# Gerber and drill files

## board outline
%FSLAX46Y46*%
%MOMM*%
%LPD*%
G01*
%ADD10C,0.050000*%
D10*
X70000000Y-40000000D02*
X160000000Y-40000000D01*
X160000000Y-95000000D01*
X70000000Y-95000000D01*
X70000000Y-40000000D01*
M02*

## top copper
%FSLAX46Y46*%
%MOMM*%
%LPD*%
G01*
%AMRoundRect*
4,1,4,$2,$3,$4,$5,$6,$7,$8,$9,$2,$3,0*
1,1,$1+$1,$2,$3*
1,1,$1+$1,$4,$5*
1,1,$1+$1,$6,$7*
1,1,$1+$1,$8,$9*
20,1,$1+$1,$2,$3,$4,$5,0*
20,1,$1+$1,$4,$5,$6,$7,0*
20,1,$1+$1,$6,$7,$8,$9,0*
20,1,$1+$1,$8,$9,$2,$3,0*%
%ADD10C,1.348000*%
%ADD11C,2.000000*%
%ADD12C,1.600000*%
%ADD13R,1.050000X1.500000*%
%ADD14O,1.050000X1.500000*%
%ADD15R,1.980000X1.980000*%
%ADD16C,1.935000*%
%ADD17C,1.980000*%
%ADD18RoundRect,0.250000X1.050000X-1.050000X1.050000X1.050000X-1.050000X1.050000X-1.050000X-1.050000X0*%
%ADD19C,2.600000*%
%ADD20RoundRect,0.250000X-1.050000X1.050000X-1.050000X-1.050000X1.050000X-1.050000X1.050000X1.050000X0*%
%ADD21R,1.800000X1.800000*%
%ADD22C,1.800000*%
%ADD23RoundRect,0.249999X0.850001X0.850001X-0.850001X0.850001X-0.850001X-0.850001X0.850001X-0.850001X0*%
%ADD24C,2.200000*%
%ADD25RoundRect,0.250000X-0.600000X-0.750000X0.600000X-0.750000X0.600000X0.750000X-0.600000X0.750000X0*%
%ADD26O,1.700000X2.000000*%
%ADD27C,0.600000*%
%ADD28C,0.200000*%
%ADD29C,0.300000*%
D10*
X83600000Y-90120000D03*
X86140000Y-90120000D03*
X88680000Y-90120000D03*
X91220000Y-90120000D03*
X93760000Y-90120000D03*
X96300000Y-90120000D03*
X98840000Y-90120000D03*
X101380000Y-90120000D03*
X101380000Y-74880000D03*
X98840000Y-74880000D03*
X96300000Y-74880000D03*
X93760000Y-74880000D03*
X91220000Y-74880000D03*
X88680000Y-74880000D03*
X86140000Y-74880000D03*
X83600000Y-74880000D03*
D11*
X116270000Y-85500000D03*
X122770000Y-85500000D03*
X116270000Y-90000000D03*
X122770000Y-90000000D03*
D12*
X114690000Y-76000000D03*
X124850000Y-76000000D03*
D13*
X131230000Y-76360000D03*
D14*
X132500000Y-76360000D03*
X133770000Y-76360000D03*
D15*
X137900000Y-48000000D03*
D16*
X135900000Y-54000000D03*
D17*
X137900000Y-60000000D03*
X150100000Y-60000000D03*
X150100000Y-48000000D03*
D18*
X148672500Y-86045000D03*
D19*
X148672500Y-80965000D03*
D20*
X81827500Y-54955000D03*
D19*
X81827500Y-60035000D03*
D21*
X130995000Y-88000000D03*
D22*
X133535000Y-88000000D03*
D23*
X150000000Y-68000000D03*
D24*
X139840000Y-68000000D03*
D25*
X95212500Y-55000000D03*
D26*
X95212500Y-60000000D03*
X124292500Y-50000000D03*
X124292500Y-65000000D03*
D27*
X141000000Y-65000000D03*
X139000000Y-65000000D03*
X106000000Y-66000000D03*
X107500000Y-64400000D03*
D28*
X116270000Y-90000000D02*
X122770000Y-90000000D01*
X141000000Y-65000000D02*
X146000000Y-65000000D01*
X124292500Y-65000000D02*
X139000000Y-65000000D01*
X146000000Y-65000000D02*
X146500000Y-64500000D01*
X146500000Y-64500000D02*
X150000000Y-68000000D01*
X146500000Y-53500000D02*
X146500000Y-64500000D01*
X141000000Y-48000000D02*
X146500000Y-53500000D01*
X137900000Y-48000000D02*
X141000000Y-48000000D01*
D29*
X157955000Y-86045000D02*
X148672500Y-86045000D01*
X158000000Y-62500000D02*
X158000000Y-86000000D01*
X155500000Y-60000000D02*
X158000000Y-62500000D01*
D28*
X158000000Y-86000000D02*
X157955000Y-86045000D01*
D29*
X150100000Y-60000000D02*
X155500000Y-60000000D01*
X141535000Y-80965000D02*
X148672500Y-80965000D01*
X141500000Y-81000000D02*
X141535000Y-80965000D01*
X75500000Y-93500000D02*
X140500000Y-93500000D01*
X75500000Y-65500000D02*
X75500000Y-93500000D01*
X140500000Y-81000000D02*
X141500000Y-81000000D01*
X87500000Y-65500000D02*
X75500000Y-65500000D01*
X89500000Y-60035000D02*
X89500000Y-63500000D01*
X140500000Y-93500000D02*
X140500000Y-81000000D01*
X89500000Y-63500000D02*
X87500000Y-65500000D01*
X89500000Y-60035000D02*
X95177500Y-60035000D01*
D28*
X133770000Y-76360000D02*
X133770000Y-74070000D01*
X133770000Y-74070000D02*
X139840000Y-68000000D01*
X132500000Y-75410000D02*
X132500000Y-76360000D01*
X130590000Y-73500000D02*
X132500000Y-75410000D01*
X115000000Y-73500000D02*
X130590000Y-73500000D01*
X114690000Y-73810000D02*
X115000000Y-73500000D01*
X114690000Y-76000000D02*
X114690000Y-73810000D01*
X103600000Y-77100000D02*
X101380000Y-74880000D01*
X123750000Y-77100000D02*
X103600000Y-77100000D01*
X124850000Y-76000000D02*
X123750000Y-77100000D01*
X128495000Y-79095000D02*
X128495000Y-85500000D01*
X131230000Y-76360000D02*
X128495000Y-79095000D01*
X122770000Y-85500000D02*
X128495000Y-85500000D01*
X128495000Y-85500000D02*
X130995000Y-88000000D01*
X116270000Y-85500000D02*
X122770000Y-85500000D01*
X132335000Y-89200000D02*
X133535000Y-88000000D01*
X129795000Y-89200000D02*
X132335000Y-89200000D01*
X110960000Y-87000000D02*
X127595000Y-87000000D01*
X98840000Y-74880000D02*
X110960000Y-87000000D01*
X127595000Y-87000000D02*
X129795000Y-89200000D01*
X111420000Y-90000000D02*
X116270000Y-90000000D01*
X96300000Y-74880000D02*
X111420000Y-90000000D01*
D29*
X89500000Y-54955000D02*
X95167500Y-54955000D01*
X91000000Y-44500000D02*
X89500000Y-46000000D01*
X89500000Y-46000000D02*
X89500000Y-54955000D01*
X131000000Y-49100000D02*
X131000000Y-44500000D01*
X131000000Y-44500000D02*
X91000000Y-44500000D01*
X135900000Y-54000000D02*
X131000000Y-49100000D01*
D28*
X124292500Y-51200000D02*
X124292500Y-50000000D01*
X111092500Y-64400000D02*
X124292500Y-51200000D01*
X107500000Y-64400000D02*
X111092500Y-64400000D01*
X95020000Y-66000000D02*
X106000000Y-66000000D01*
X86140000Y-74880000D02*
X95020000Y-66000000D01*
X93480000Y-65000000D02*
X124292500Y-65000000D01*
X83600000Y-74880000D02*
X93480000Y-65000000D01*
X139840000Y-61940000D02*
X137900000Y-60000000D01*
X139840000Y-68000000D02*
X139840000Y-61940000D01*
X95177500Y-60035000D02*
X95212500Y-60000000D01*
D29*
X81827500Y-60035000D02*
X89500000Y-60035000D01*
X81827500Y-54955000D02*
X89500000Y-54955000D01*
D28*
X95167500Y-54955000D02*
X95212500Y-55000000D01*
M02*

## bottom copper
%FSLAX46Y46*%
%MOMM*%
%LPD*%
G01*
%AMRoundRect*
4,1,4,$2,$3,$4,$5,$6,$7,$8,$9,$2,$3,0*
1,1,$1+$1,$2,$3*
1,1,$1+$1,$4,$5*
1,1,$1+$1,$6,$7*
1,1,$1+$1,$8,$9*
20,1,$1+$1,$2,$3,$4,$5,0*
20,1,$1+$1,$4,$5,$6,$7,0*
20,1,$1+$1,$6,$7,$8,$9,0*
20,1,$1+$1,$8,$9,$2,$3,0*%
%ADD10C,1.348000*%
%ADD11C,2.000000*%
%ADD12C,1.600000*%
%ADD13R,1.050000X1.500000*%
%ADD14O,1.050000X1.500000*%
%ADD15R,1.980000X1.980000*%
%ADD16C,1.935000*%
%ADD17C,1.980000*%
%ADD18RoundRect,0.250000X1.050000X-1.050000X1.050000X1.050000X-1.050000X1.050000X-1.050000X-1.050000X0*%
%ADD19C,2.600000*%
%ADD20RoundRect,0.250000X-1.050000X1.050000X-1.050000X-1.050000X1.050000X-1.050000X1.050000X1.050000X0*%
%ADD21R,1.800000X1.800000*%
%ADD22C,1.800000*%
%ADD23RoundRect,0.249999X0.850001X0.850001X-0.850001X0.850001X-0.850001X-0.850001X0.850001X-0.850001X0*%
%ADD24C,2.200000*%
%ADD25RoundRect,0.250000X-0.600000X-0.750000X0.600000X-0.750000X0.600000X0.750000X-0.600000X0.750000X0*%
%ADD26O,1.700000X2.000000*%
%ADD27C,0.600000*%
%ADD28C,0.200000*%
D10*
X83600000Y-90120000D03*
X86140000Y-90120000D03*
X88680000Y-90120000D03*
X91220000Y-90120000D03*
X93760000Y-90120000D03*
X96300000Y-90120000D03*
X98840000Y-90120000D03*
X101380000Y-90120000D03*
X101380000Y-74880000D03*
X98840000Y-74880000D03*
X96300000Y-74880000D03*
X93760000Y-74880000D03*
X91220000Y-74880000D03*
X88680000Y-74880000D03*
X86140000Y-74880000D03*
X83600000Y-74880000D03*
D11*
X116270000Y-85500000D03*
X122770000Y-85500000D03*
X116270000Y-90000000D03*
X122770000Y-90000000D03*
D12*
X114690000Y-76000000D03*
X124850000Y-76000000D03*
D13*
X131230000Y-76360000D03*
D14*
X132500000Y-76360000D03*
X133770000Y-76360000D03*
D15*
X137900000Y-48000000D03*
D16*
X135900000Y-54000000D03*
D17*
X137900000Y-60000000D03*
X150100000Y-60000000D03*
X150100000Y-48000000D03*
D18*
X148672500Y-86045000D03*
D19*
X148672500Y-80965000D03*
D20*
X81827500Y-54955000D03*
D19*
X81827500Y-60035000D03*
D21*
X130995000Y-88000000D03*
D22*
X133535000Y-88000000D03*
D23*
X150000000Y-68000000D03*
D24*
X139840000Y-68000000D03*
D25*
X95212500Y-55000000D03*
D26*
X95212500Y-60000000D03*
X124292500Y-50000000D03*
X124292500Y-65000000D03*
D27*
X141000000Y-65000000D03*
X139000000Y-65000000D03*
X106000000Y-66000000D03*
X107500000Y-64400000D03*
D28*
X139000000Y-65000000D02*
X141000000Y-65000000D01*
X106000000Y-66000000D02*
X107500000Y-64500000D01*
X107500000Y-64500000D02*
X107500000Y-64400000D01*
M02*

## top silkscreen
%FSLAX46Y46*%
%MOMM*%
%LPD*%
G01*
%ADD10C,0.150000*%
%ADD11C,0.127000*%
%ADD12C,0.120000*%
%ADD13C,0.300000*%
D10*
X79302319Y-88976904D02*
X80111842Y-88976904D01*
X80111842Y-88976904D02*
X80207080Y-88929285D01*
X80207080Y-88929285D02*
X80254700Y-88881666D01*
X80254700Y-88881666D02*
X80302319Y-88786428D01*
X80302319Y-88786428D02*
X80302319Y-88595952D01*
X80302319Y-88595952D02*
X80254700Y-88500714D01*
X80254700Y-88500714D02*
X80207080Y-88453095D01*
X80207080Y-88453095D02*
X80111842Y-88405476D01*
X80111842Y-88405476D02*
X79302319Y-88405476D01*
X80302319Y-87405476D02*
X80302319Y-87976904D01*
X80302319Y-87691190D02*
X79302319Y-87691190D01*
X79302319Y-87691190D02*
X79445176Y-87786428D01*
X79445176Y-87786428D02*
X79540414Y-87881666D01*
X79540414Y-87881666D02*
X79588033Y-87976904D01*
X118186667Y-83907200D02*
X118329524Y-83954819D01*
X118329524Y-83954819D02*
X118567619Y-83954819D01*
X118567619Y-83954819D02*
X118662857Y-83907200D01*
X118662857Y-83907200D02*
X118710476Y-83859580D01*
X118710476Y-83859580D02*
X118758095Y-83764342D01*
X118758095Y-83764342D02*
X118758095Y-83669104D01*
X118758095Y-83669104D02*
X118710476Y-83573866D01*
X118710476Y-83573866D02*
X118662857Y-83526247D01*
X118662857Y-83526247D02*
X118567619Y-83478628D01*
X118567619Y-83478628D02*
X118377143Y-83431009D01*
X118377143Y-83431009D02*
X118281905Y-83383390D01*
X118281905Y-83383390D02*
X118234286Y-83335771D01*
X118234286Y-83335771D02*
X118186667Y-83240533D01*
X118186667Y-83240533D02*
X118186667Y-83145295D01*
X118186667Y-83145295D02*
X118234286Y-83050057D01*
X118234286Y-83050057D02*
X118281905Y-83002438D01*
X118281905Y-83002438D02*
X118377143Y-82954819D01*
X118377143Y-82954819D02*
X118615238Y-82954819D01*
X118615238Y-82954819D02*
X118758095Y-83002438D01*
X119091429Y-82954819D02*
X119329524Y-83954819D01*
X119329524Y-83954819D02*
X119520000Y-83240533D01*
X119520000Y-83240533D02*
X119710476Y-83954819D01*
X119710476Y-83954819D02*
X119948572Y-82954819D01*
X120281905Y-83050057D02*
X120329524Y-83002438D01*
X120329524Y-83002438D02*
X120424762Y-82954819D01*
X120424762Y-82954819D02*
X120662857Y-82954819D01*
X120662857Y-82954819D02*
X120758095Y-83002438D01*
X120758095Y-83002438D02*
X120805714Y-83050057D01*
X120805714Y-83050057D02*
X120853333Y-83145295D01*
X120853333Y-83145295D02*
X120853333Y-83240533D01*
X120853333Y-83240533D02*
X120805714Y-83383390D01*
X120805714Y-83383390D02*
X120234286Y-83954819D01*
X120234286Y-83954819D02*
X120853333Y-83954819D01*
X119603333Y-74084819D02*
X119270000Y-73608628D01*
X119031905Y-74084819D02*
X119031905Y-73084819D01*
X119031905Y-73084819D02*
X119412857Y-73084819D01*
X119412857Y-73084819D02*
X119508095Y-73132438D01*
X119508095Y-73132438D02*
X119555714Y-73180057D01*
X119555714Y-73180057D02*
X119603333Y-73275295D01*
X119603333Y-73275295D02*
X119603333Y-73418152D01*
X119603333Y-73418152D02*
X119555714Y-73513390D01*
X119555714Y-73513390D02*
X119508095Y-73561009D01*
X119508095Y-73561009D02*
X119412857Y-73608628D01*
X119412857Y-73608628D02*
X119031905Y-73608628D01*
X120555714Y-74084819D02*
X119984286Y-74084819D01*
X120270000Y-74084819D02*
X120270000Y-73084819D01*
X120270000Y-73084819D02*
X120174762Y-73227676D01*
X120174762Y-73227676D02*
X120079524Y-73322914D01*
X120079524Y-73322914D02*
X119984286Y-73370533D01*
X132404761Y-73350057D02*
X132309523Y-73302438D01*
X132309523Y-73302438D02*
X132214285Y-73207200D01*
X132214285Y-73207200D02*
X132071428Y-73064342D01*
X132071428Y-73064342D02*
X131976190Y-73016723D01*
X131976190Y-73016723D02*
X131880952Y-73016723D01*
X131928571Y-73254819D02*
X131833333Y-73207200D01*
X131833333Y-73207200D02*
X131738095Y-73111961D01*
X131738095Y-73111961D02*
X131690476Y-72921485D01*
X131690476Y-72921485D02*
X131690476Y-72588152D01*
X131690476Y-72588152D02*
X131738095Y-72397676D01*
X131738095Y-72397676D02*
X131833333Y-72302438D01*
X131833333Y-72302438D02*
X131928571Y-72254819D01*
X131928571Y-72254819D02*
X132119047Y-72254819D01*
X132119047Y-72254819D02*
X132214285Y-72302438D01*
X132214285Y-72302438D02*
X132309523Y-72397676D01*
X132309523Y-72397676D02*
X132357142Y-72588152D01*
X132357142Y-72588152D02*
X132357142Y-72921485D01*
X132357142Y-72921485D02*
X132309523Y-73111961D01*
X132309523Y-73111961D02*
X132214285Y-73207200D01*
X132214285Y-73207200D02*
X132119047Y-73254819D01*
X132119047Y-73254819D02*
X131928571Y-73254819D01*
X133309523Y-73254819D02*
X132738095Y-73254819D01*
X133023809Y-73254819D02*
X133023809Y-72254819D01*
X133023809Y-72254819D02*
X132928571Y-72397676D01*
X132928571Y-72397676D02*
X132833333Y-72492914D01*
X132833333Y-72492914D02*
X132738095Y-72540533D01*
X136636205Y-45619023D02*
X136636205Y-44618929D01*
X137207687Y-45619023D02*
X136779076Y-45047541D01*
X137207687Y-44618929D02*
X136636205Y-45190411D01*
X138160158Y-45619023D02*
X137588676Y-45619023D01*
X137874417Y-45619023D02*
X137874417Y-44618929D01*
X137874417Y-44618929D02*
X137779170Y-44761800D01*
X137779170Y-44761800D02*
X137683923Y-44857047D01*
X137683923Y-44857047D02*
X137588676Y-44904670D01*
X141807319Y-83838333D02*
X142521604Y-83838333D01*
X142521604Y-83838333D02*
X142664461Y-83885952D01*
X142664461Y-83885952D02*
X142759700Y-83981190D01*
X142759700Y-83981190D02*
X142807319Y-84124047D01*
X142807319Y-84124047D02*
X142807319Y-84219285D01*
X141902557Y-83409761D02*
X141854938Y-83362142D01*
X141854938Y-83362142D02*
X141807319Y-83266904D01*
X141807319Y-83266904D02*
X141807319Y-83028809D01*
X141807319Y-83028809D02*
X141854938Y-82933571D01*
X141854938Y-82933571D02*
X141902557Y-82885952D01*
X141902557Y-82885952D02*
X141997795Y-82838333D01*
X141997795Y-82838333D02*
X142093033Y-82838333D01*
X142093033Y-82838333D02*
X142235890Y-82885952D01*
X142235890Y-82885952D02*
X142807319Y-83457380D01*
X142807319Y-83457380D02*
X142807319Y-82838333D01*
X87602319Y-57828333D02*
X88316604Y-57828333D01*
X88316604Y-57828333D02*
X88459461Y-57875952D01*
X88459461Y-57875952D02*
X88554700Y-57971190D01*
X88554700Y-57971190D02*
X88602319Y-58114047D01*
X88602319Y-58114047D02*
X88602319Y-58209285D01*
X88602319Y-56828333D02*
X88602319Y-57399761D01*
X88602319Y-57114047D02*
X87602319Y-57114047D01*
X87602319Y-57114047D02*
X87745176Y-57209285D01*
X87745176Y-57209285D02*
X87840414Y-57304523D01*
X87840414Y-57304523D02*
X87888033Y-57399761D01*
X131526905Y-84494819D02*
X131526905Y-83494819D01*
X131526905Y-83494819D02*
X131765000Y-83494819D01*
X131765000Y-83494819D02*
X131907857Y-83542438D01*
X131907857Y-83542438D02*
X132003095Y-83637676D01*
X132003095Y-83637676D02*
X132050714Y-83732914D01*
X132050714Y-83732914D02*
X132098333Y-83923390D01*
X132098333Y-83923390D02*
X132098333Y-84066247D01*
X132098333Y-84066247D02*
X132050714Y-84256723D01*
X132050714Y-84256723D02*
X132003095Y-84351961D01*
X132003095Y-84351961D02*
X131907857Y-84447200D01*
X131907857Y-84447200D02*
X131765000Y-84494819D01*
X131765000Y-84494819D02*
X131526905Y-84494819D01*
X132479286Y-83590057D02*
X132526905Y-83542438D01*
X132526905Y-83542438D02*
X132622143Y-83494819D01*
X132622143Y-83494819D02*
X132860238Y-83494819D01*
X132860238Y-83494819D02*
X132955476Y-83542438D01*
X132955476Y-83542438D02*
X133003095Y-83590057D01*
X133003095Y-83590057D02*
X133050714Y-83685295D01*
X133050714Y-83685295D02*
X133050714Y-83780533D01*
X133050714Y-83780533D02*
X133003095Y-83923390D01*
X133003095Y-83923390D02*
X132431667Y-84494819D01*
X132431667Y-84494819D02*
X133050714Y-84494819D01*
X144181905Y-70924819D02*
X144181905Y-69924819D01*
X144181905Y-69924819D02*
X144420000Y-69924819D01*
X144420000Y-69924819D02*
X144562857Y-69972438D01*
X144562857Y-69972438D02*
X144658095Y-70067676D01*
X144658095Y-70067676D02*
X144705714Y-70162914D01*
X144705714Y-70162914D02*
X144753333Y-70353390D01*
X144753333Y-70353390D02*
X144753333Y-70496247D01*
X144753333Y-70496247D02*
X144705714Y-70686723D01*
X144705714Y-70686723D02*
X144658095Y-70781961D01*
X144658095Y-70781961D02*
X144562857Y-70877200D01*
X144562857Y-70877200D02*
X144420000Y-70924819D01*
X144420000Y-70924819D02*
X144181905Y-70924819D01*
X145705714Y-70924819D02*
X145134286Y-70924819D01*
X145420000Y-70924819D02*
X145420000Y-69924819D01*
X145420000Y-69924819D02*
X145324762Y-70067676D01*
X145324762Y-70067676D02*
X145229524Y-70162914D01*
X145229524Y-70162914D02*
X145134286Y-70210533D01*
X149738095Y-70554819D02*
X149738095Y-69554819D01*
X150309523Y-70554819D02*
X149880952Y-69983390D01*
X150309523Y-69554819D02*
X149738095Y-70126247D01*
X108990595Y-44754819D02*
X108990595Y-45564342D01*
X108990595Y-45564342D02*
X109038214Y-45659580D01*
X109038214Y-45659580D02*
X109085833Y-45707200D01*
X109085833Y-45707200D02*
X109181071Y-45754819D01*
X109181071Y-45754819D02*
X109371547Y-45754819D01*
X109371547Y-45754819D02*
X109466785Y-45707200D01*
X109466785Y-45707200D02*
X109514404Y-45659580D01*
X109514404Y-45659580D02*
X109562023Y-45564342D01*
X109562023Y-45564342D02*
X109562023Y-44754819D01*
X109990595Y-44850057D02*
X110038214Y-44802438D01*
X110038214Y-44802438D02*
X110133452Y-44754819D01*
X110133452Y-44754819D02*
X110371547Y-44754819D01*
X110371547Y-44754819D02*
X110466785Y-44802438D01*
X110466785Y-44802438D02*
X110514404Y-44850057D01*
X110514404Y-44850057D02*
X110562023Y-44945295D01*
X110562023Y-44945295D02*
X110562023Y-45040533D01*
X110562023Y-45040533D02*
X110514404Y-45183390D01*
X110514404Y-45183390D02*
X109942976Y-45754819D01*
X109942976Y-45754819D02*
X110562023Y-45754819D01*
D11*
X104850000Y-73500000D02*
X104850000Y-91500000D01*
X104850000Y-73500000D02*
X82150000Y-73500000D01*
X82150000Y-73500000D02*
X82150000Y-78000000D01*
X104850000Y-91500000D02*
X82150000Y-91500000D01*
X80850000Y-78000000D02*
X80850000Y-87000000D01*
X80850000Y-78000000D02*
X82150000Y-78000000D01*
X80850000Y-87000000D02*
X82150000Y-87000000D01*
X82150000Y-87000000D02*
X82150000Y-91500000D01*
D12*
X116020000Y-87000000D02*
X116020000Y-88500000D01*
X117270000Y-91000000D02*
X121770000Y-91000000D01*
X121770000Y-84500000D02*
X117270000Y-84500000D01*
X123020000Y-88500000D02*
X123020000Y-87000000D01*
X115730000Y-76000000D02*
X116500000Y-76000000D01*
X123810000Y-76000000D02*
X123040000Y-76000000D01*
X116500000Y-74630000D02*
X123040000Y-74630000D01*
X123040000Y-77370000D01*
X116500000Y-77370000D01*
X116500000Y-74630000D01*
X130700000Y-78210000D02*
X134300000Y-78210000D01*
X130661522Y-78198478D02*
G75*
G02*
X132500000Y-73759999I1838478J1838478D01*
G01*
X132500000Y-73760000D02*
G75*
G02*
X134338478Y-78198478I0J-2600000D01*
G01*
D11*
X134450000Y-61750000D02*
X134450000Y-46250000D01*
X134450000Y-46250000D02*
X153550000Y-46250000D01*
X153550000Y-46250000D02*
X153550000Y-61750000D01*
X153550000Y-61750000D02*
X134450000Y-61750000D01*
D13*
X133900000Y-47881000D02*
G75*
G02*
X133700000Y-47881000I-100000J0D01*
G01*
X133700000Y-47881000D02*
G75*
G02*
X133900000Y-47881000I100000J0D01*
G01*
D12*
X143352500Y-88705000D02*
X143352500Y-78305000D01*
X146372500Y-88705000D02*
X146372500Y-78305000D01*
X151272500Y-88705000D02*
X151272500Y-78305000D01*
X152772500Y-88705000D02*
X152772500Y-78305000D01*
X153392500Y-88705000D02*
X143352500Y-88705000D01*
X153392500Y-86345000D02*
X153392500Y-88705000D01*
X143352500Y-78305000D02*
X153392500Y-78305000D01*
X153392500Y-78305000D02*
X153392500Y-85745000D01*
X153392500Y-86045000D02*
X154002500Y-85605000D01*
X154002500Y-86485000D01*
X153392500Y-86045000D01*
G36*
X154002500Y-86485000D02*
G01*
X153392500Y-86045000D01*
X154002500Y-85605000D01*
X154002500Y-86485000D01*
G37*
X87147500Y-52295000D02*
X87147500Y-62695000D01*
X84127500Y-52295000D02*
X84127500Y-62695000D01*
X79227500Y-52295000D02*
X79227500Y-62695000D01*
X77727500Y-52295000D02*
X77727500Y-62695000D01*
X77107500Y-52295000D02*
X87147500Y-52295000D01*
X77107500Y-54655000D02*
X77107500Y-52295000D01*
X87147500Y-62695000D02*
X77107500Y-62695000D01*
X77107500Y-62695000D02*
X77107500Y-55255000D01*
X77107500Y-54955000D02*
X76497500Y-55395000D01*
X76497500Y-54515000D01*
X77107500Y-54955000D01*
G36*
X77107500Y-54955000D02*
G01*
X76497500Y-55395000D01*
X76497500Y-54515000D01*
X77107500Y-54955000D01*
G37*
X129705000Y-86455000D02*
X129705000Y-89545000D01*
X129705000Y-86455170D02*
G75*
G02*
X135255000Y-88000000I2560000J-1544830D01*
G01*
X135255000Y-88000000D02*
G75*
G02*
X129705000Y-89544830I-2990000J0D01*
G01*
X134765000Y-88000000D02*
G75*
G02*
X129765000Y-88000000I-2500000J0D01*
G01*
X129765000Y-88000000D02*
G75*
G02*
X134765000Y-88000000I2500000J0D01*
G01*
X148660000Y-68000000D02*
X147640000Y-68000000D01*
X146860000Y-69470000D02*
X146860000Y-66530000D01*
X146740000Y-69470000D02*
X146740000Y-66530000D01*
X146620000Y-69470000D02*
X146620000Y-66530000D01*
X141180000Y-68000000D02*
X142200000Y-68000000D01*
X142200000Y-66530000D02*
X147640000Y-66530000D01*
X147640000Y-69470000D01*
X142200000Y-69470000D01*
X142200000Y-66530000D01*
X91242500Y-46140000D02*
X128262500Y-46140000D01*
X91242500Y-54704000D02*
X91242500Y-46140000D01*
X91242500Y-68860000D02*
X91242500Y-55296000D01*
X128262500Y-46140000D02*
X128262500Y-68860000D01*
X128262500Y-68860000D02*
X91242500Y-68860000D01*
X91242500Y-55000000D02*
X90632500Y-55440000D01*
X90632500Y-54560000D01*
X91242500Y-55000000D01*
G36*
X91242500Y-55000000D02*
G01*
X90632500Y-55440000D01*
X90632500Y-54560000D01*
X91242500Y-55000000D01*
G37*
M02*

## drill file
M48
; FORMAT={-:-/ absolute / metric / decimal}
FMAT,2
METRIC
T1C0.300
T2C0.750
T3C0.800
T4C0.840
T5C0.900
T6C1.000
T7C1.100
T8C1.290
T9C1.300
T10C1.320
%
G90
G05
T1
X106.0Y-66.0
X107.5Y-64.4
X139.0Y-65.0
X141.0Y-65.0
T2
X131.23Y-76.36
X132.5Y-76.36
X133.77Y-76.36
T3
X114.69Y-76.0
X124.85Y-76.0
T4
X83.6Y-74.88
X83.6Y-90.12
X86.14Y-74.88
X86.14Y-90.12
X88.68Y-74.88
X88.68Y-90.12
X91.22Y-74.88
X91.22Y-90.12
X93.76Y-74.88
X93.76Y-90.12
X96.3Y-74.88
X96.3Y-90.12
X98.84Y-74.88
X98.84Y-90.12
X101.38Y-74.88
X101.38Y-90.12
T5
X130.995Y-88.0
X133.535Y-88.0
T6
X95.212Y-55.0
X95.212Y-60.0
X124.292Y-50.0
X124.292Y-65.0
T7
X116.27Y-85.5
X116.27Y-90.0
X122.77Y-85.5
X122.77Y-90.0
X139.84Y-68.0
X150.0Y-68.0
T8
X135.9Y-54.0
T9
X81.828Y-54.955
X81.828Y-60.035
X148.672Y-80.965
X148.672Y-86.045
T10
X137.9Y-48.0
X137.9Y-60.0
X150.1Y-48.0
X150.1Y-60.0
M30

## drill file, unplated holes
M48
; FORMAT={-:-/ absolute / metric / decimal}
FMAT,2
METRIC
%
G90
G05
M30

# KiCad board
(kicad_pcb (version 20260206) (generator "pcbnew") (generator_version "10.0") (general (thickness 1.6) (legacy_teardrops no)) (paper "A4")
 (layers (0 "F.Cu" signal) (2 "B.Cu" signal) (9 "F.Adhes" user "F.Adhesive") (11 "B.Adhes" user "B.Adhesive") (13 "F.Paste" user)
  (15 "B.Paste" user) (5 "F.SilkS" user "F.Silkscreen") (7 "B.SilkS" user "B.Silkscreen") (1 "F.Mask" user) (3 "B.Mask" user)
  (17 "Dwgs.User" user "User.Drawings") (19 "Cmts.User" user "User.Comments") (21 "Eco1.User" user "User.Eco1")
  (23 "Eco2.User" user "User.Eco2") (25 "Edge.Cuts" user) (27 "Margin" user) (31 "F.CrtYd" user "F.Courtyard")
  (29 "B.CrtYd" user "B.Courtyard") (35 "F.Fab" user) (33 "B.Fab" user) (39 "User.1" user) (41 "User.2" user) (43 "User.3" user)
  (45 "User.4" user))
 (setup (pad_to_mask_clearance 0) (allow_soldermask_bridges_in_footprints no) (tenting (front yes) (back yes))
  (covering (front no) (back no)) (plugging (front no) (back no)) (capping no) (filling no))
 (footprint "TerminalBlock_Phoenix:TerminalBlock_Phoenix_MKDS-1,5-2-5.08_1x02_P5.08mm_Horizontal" (layer "F.Cu") (at 148.6725 86.045 90)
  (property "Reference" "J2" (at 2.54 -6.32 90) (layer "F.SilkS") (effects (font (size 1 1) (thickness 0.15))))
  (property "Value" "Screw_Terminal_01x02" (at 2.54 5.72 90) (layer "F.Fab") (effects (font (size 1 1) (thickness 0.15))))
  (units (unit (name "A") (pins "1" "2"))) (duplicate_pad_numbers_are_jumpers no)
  (fp_line (start 7.74 -5.32) (end 7.74 4.72) (stroke (width 0.12) (type solid)) (layer "F.SilkS"))
  (fp_line (start -2.66 -5.32) (end 7.74 -5.32) (stroke (width 0.12) (type solid)) (layer "F.SilkS"))
  (fp_line (start -2.66 -2.3) (end 7.74 -2.3) (stroke (width 0.12) (type solid)) (layer "F.SilkS"))
  (fp_line (start -2.66 2.6) (end 7.74 2.6) (stroke (width 0.12) (type solid)) (layer "F.SilkS"))
  (fp_line (start -2.66 4.1) (end 7.74 4.1) (stroke (width 0.12) (type solid)) (layer "F.SilkS"))
  (fp_line (start 7.74 4.72) (end 0.3 4.72) (stroke (width 0.12) (type solid)) (layer "F.SilkS"))
  (fp_line (start -0.3 4.72) (end -2.66 4.72) (stroke (width 0.12) (type solid)) (layer "F.SilkS"))
  (fp_line (start -2.66 4.72) (end -2.66 -5.32) (stroke (width 0.12) (type solid)) (layer "F.SilkS"))
  (fp_poly (pts (xy 0 4.72) (xy 0.44 5.33) (xy -0.44 5.33)) (stroke (width 0.12) (type solid)) (fill yes) (layer "F.SilkS"))
  (pad "1" thru_hole roundrect (at 0 0 90) (size 2.6 2.6) (drill 1.3) (layers "*.Cu" "*.Mask") (remove_unused_layers no)
   (roundrect_rratio 0.096154) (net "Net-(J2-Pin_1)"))
  (pad "2" thru_hole circle (at 5.08 0 90) (size 2.6 2.6) (drill 1.3) (layers "*.Cu" "*.Mask") (remove_unused_layers no)
   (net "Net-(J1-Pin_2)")))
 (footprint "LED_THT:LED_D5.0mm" (layer "F.Cu") (at 130.995 88)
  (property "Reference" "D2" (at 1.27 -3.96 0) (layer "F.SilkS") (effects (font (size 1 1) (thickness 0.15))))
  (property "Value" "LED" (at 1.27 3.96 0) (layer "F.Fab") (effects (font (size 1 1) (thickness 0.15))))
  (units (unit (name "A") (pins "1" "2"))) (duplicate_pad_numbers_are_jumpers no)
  (fp_line (start -1.29 -1.545) (end -1.29 1.545) (stroke (width 0.12) (type solid)) (layer "F.SilkS"))
  (fp_arc (start -1.29 -1.54483) (mid 2.071779 -2.880495) (end 4.26 0) (stroke (width 0.12) (type solid)) (layer "F.SilkS"))
  (fp_arc (start 4.26 0) (mid 2.071779 2.880495) (end -1.29 1.54483) (stroke (width 0.12) (type solid)) (layer "F.SilkS"))
  (fp_circle (center 1.27 0) (end 3.77 0) (stroke (width 0.12) (type solid)) (fill no) (layer "F.SilkS"))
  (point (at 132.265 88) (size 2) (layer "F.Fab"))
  (pad "1" thru_hole rect (at 0 0) (size 1.8 1.8) (drill 0.9) (layers "*.Cu" "*.Mask") (remove_unused_layers no) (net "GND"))
  (pad "2" thru_hole circle (at 2.54 0) (size 1.8 1.8) (drill 0.9) (layers "*.Cu" "*.Mask") (remove_unused_layers no) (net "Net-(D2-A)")))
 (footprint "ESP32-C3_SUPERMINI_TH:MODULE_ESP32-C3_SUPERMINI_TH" (layer "F.Cu") (at 93.5 82.5 90)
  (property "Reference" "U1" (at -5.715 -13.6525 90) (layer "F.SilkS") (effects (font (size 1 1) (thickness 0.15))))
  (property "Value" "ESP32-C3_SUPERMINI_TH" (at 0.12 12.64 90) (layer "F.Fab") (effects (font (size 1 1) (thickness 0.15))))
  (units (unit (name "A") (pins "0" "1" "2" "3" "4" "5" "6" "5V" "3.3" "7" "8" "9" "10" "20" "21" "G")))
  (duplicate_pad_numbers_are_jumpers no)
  (fp_line (start 4.5 -12.65) (end -4.5 -12.65) (stroke (width 0.127) (type solid)) (layer "F.SilkS"))
  (fp_line (start 4.5 -12.65) (end 4.5 -11.35) (stroke (width 0.127) (type solid)) (layer "F.SilkS"))
  (fp_line (start -4.5 -12.65) (end -4.5 -11.35) (stroke (width 0.127) (type solid)) (layer "F.SilkS"))
  (fp_line (start 9 -11.35) (end 4.5 -11.35) (stroke (width 0.127) (type solid)) (layer "F.SilkS"))
  (fp_line (start -4.5 -11.35) (end -9 -11.35) (stroke (width 0.127) (type solid)) (layer "F.SilkS"))
  (fp_line (start 9 11.35) (end 9 -11.35) (stroke (width 0.127) (type solid)) (layer "F.SilkS"))
  (fp_line (start 9 11.35) (end -9 11.35) (stroke (width 0.127) (type solid)) (layer "F.SilkS"))
  (fp_line (start -9 11.35) (end -9 -11.35) (stroke (width 0.127) (type solid)) (layer "F.SilkS"))
  (pad "0" thru_hole circle (at 7.62 7.88 90) (size 1.348 1.348) (drill 0.84) (layers "*.Cu" "*.Mask") (remove_unused_layers no)
   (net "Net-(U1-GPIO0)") (solder_mask_margin 0.102))
  (pad "1" thru_hole circle (at 7.62 5.34 90) (size 1.348 1.348) (drill 0.84) (layers "*.Cu" "*.Mask") (remove_unused_layers no)
   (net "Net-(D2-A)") (solder_mask_margin 0.102))
  (pad "2" thru_hole circle (at 7.62 2.8 90) (size 1.348 1.348) (drill 0.84) (layers "*.Cu" "*.Mask") (remove_unused_layers no)
   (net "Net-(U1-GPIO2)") (solder_mask_margin 0.102))
  (pad "3" thru_hole circle (at 7.62 0.26 90) (size 1.348 1.348) (drill 0.84) (layers "*.Cu" "*.Mask") (remove_unused_layers no)
   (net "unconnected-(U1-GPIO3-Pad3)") (solder_mask_margin 0.102))
  (pad "3.3" thru_hole circle (at 7.62 -4.82 90) (size 1.348 1.348) (drill 0.84) (layers "*.Cu" "*.Mask") (remove_unused_layers no)
   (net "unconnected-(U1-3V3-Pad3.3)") (solder_mask_margin 0.102))
  (pad "4" thru_hole circle (at 7.62 -2.28 90) (size 1.348 1.348) (drill 0.84) (layers "*.Cu" "*.Mask") (remove_unused_layers no)
   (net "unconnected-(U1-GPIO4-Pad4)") (solder_mask_margin 0.102))
  (pad "5" thru_hole circle (at -7.62 -9.9 90) (size 1.348 1.348) (drill 0.84) (layers "*.Cu" "*.Mask") (remove_unused_layers no)
   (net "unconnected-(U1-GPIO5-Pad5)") (solder_mask_margin 0.102))
  (pad "5V" thru_hole circle (at 7.62 -9.9 90) (size 1.348 1.348) (drill 0.84) (layers "*.Cu" "*.Mask") (remove_unused_layers no)
   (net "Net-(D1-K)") (solder_mask_margin 0.102))
  (pad "6" thru_hole circle (at -7.62 -7.36 90) (size 1.348 1.348) (drill 0.84) (layers "*.Cu" "*.Mask") (remove_unused_layers no)
   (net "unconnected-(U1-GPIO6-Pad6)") (solder_mask_margin 0.102))
  (pad "7" thru_hole circle (at -7.62 -4.82 90) (size 1.348 1.348) (drill 0.84) (layers "*.Cu" "*.Mask") (remove_unused_layers no)
   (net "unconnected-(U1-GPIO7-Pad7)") (solder_mask_margin 0.102))
  (pad "8" thru_hole circle (at -7.62 -2.28 90) (size 1.348 1.348) (drill 0.84) (layers "*.Cu" "*.Mask") (remove_unused_layers no)
   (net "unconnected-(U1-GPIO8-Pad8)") (solder_mask_margin 0.102))
  (pad "9" thru_hole circle (at -7.62 0.26 90) (size 1.348 1.348) (drill 0.84) (layers "*.Cu" "*.Mask") (remove_unused_layers no)
   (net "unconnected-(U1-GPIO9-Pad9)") (solder_mask_margin 0.102))
  (pad "10" thru_hole circle (at -7.62 2.8 90) (size 1.348 1.348) (drill 0.84) (layers "*.Cu" "*.Mask") (remove_unused_layers no)
   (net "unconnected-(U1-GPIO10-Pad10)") (solder_mask_margin 0.102))
  (pad "20" thru_hole circle (at -7.62 5.34 90) (size 1.348 1.348) (drill 0.84) (layers "*.Cu" "*.Mask") (remove_unused_layers no)
   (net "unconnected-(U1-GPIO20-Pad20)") (solder_mask_margin 0.102))
  (pad "21" thru_hole circle (at -7.62 7.88 90) (size 1.348 1.348) (drill 0.84) (layers "*.Cu" "*.Mask") (remove_unused_layers no)
   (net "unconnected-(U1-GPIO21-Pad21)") (solder_mask_margin 0.102))
  (pad "G" thru_hole circle (at 7.62 -7.36 90) (size 1.348 1.348) (drill 0.84) (layers "*.Cu" "*.Mask") (remove_unused_layers no)
   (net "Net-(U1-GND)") (solder_mask_margin 0.102)))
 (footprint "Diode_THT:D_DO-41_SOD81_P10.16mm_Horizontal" (layer "F.Cu") (at 150 68 180)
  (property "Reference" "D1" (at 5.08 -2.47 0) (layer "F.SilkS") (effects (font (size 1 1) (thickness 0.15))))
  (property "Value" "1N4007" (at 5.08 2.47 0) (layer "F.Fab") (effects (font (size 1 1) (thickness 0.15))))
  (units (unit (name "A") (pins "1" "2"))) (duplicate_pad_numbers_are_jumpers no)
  (fp_line (start 8.82 0) (end 7.8 0) (stroke (width 0.12) (type solid)) (layer "F.SilkS"))
  (fp_line (start 3.38 -1.47) (end 3.38 1.47) (stroke (width 0.12) (type solid)) (layer "F.SilkS"))
  (fp_line (start 3.26 -1.47) (end 3.26 1.47) (stroke (width 0.12) (type solid)) (layer "F.SilkS"))
  (fp_line (start 3.14 -1.47) (end 3.14 1.47) (stroke (width 0.12) (type solid)) (layer "F.SilkS"))
  (fp_line (start 1.34 0) (end 2.36 0) (stroke (width 0.12) (type solid)) (layer "F.SilkS"))
  (fp_rect (start 2.36 -1.47) (end 7.8 1.47) (stroke (width 0.12) (type solid)) (fill no) (layer "F.SilkS"))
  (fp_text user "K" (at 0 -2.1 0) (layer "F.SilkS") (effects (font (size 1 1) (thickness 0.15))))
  (pad "1" thru_hole roundrect (at 0 0 180) (size 2.2 2.2) (drill 1.1) (layers "*.Cu" "*.Mask") (remove_unused_layers no)
   (roundrect_rratio 0.113636) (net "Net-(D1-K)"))
  (pad "2" thru_hole circle (at 10.16 0 180) (size 2.2 2.2) (drill 1.1) (layers "*.Cu" "*.Mask") (remove_unused_layers no)
   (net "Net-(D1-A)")))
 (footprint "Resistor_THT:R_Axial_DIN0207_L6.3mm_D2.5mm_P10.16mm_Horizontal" (layer "F.Cu") (at 114.69 76)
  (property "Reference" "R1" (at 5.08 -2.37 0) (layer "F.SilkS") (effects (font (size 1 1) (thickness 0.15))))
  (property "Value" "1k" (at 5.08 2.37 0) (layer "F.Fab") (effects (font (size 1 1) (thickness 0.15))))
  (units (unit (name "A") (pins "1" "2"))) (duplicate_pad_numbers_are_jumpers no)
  (fp_line (start 1.04 0) (end 1.81 0) (stroke (width 0.12) (type solid)) (layer "F.SilkS"))
  (fp_line (start 9.12 0) (end 8.35 0) (stroke (width 0.12) (type solid)) (layer "F.SilkS"))
  (fp_rect (start 1.81 -1.37) (end 8.35 1.37) (stroke (width 0.12) (type solid)) (fill no) (layer "F.SilkS"))
  (pad "1" thru_hole circle (at 0 0) (size 1.6 1.6) (drill 0.8) (layers "*.Cu" "*.Mask") (remove_unused_layers no) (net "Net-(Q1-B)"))
  (pad "2" thru_hole circle (at 10.16 0) (size 1.6 1.6) (drill 0.8) (layers "*.Cu" "*.Mask") (remove_unused_layers no)
   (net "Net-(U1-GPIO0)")))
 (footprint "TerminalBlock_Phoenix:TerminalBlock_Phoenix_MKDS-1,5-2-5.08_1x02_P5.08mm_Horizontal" (layer "F.Cu") (at 81.8275 54.955 -90)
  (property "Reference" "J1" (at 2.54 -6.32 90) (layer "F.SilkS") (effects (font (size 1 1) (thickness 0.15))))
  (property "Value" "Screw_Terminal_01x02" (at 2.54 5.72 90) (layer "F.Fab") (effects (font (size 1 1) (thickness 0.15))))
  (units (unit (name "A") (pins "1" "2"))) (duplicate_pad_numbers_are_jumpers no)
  (fp_line (start -2.66 4.72) (end -2.66 -5.32) (stroke (width 0.12) (type solid)) (layer "F.SilkS"))
  (fp_line (start -0.3 4.72) (end -2.66 4.72) (stroke (width 0.12) (type solid)) (layer "F.SilkS"))
  (fp_line (start 7.74 4.72) (end 0.3 4.72) (stroke (width 0.12) (type solid)) (layer "F.SilkS"))
  (fp_line (start -2.66 4.1) (end 7.74 4.1) (stroke (width 0.12) (type solid)) (layer "F.SilkS"))
  (fp_line (start -2.66 2.6) (end 7.74 2.6) (stroke (width 0.12) (type solid)) (layer "F.SilkS"))
  (fp_line (start -2.66 -2.3) (end 7.74 -2.3) (stroke (width 0.12) (type solid)) (layer "F.SilkS"))
  (fp_line (start -2.66 -5.32) (end 7.74 -5.32) (stroke (width 0.12) (type solid)) (layer "F.SilkS"))
  (fp_line (start 7.74 -5.32) (end 7.74 4.72) (stroke (width 0.12) (type solid)) (layer "F.SilkS"))
  (fp_poly (pts (xy 0 4.72) (xy 0.44 5.33) (xy -0.44 5.33)) (stroke (width 0.12) (type solid)) (fill yes) (layer "F.SilkS"))
  (pad "1" thru_hole roundrect (at 0 0 270) (size 2.6 2.6) (drill 1.3) (layers "*.Cu" "*.Mask") (remove_unused_layers no)
   (roundrect_rratio 0.096154) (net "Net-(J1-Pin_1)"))
  (pad "2" thru_hole circle (at 5.08 0 270) (size 2.6 2.6) (drill 1.3) (layers "*.Cu" "*.Mask") (remove_unused_layers no)
   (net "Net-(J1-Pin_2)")))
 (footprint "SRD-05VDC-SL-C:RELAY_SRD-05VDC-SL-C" (layer "F.Cu") (at 144 54)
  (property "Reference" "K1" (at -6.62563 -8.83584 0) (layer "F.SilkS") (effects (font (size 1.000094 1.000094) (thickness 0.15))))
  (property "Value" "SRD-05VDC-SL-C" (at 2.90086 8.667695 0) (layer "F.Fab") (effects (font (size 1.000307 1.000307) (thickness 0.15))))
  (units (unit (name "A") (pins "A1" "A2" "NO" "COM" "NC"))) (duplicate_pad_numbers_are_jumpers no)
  (fp_line (start -9.55 -7.75) (end 9.55 -7.75) (stroke (width 0.127) (type solid)) (layer "F.SilkS"))
  (fp_line (start -9.55 7.75) (end -9.55 -7.75) (stroke (width 0.127) (type solid)) (layer "F.SilkS"))
  (fp_line (start 9.55 -7.75) (end 9.55 7.75) (stroke (width 0.127) (type solid)) (layer "F.SilkS"))
  (fp_line (start 9.55 7.75) (end -9.55 7.75) (stroke (width 0.127) (type solid)) (layer "F.SilkS"))
  (fp_circle (center -10.2 -6.119) (end -10.1 -6.119) (stroke (width 0.3) (type solid)) (fill no) (layer "F.SilkS"))
  (pad "A1" thru_hole rect (at -6.1 -6) (size 1.98 1.98) (drill 1.32) (layers "*.Cu" "*.Mask") (remove_unused_layers no) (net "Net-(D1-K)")
   (solder_mask_margin 0.102))
  (pad "A2" thru_hole circle (at -6.1 6) (size 1.98 1.98) (drill 1.32) (layers "*.Cu" "*.Mask") (remove_unused_layers no) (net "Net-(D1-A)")
   (solder_mask_margin 0.102))
  (pad "COM" thru_hole circle (at -8.1 0) (size 1.935 1.935) (drill 1.29) (layers "*.Cu" "*.Mask") (remove_unused_layers no)
   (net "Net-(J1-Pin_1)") (solder_mask_margin 0.102))
  (pad "NC" thru_hole circle (at 6.1 -6) (size 1.98 1.98) (drill 1.32) (layers "*.Cu" "*.Mask") (remove_unused_layers no)
   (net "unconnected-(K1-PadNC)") (solder_mask_margin 0.102))
  (pad "NO" thru_hole circle (at 6.1 6) (size 1.98 1.98) (drill 1.32) (layers "*.Cu" "*.Mask") (remove_unused_layers no)
   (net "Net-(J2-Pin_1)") (solder_mask_margin 0.102)))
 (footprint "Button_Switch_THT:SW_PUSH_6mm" (layer "F.Cu") (at 116.27 85.5)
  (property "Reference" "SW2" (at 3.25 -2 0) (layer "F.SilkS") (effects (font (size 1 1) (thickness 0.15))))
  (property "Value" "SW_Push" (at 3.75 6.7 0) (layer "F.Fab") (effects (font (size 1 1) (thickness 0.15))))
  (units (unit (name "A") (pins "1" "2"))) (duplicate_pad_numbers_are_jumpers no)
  (fp_line (start -0.25 1.5) (end -0.25 3) (stroke (width 0.12) (type solid)) (layer "F.SilkS"))
  (fp_line (start 1 5.5) (end 5.5 5.5) (stroke (width 0.12) (type solid)) (layer "F.SilkS"))
  (fp_line (start 5.5 -1) (end 1 -1) (stroke (width 0.12) (type solid)) (layer "F.SilkS"))
  (fp_line (start 6.75 3) (end 6.75 1.5) (stroke (width 0.12) (type solid)) (layer "F.SilkS"))
  (pad "1" thru_hole circle (at 0 0 90) (size 2 2) (drill 1.1) (layers "*.Cu" "*.Mask") (remove_unused_layers no) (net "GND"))
  (pad "1" thru_hole circle (at 6.5 0 90) (size 2 2) (drill 1.1) (layers "*.Cu" "*.Mask") (remove_unused_layers no) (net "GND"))
  (pad "2" thru_hole circle (at 0 4.5 90) (size 2 2) (drill 1.1) (layers "*.Cu" "*.Mask") (remove_unused_layers no) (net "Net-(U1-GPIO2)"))
  (pad "2" thru_hole circle (at 6.5 4.5 90) (size 2 2) (drill 1.1) (layers "*.Cu" "*.Mask") (remove_unused_layers no) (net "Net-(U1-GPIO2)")))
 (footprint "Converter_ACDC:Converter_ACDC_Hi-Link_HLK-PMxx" (layer "F.Cu") (at 95.2125 55)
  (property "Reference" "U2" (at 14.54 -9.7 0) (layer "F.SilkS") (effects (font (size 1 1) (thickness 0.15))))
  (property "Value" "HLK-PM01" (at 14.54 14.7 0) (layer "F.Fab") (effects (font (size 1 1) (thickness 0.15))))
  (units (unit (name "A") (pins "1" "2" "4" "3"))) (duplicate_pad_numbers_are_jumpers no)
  (fp_line (start -3.97 -8.86) (end 33.05 -8.86) (stroke (width 0.12) (type solid)) (layer "F.SilkS"))
  (fp_line (start -3.97 -0.296) (end -3.97 -8.86) (stroke (width 0.12) (type solid)) (layer "F.SilkS"))
  (fp_line (start -3.97 13.86) (end -3.97 0.296) (stroke (width 0.12) (type solid)) (layer "F.SilkS"))
  (fp_line (start 33.05 -8.86) (end 33.05 13.86) (stroke (width 0.12) (type solid)) (layer "F.SilkS"))
  (fp_line (start 33.05 13.86) (end -3.97 13.86) (stroke (width 0.12) (type solid)) (layer "F.SilkS"))
  (fp_poly (pts (xy -3.97 0) (xy -4.58 0.44) (xy -4.58 -0.44)) (stroke (width 0.12) (type solid)) (fill yes) (layer "F.SilkS"))
  (pad "1" thru_hole roundrect (at 0 0) (size 1.7 2) (drill 1) (layers "*.Cu" "*.Mask") (remove_unused_layers no)
   (roundrect_rratio 0.147059) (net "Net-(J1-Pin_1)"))
  (pad "2" thru_hole oval (at 0 5) (size 1.7 2) (drill 1) (layers "*.Cu" "*.Mask") (remove_unused_layers no) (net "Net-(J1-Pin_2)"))
  (pad "3" thru_hole oval (at 29.08 -5) (size 1.7 2) (drill 1) (layers "*.Cu" "*.Mask") (remove_unused_layers no) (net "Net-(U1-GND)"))
  (pad "4" thru_hole oval (at 29.08 10) (size 1.7 2) (drill 1) (layers "*.Cu" "*.Mask") (remove_unused_layers no) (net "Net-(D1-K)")))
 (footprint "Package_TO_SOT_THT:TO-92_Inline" (layer "F.Cu") (at 131.23 76.36)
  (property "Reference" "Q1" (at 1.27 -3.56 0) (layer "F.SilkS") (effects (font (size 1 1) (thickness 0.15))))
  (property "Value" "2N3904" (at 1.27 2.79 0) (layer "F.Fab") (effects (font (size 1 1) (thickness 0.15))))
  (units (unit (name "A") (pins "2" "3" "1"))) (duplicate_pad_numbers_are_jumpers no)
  (fp_line (start -0.53 1.85) (end 3.07 1.85) (stroke (width 0.12) (type solid)) (layer "F.SilkS"))
  (fp_arc (start -0.568478 1.838478) (mid -1.132087 -0.994977) (end 1.27 -2.6) (stroke (width 0.12) (type solid)) (layer "F.SilkS"))
  (fp_arc (start 1.27 -2.6) (mid 3.672087 -0.994977) (end 3.108478 1.838478) (stroke (width 0.12) (type solid)) (layer "F.SilkS"))
  (pad "1" thru_hole rect (at 0 0) (size 1.05 1.5) (drill 0.75) (layers "*.Cu" "*.Mask") (remove_unused_layers no) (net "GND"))
  (pad "2" thru_hole oval (at 1.27 0) (size 1.05 1.5) (drill 0.75) (layers "*.Cu" "*.Mask") (remove_unused_layers no) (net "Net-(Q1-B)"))
  (pad "3" thru_hole oval (at 2.54 0) (size 1.05 1.5) (drill 0.75) (layers "*.Cu" "*.Mask") (remove_unused_layers no) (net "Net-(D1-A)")))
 (gr_rect (start 70 40) (end 160 95) (stroke (width 0.05) (type default)) (fill no) (layer "Edge.Cuts"))
 (segment (start 83.6 74.88) (end 93.48 65) (width 0.2) (layer "F.Cu") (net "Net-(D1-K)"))
 (segment (start 146.5 64.5) (end 150 68) (width 0.2) (layer "F.Cu") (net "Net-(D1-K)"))
 (segment (start 146.5 53.5) (end 146.5 64.5) (width 0.2) (layer "F.Cu") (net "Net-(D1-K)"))
 (segment (start 93.48 65) (end 124.2925 65) (width 0.2) (layer "F.Cu") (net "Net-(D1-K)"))
 (segment (start 124.2925 65) (end 139 65) (width 0.2) (layer "F.Cu") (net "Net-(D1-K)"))
 (segment (start 141 65) (end 146 65) (width 0.2) (layer "F.Cu") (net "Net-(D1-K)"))
 (segment (start 137.9 48) (end 141 48) (width 0.2) (layer "F.Cu") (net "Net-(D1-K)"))
 (segment (start 141 48) (end 146.5 53.5) (width 0.2) (layer "F.Cu") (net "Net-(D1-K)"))
 (segment (start 146 65) (end 146.5 64.5) (width 0.2) (layer "F.Cu") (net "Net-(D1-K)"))
 (via (at 139 65) (size 0.6) (drill 0.3) (layers "F.Cu" "B.Cu") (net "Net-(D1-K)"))
 (via (at 141 65) (size 0.6) (drill 0.3) (layers "F.Cu" "B.Cu") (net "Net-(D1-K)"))
 (segment (start 139 65) (end 141 65) (width 0.2) (layer "B.Cu") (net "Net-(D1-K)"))
 (segment (start 133.77 74.07) (end 139.84 68) (width 0.2) (layer "F.Cu") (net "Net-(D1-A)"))
 (segment (start 139.84 61.94) (end 137.9 60) (width 0.2) (layer "F.Cu") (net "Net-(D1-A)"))
 (segment (start 139.84 68) (end 139.84 61.94) (width 0.2) (layer "F.Cu") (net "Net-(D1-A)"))
 (segment (start 133.77 76.36) (end 133.77 74.07) (width 0.2) (layer "F.Cu") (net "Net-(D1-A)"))
 (segment (start 122.77 85.5) (end 128.495 85.5) (width 0.2) (layer "F.Cu") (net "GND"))
 (segment (start 131.23 76.36) (end 128.495 79.095) (width 0.2) (layer "F.Cu") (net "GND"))
 (segment (start 128.495 85.5) (end 130.995 88) (width 0.2) (layer "F.Cu") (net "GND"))
 (segment (start 116.27 85.5) (end 122.77 85.5) (width 0.2) (layer "F.Cu") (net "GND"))
 (segment (start 128.495 79.095) (end 128.495 85.5) (width 0.2) (layer "F.Cu") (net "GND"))
 (segment (start 110.96 87) (end 127.595 87) (width 0.2) (layer "F.Cu") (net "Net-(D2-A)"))
 (segment (start 129.795 89.2) (end 132.335 89.2) (width 0.2) (layer "F.Cu") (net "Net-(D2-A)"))
 (segment (start 127.595 87) (end 129.795 89.2) (width 0.2) (layer "F.Cu") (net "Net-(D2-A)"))
 (segment (start 98.84 74.88) (end 110.96 87) (width 0.2) (layer "F.Cu") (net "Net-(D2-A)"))
 (segment (start 132.335 89.2) (end 133.535 88) (width 0.2) (layer "F.Cu") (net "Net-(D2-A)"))
 (segment (start 81.8275 54.955) (end 89.5 54.955) (width 0.3) (layer "F.Cu") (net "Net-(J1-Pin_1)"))
 (segment (start 131 44.5) (end 91 44.5) (width 0.3) (layer "F.Cu") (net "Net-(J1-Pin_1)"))
 (segment (start 135.9 54) (end 131 49.1) (width 0.3) (layer "F.Cu") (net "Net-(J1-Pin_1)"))
 (segment (start 89.5 54.955) (end 95.1675 54.955) (width 0.3) (layer "F.Cu") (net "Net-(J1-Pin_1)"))
 (segment (start 91 44.5) (end 89.5 46) (width 0.3) (layer "F.Cu") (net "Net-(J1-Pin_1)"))
 (segment (start 95.1675 54.955) (end 95.2125 55) (width 0.2) (layer "F.Cu") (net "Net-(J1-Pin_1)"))
 (segment (start 89.5 46) (end 89.5 54.955) (width 0.3) (layer "F.Cu") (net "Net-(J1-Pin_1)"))
 (segment (start 131 49.1) (end 131 44.5) (width 0.3) (layer "F.Cu") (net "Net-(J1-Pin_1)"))
 (segment (start 75.5 93.5) (end 140.5 93.5) (width 0.3) (layer "F.Cu") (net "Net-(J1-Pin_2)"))
 (segment (start 89.5 63.5) (end 87.5 65.5) (width 0.3) (layer "F.Cu") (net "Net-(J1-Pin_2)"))
 (segment (start 87.5 65.5) (end 75.5 65.5) (width 0.3) (layer "F.Cu") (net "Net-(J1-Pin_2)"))
 (segment (start 140.5 81) (end 141.5 81) (width 0.3) (layer "F.Cu") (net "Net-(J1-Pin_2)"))
 (segment (start 89.5 60.035) (end 95.1775 60.035) (width 0.3) (layer "F.Cu") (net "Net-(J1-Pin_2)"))
 (segment (start 141.5 81) (end 141.535 80.965) (width 0.3) (layer "F.Cu") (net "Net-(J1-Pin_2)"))
 (segment (start 141.535 80.965) (end 148.6725 80.965) (width 0.3) (layer "F.Cu") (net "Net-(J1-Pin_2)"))
 (segment (start 95.1775 60.035) (end 95.2125 60) (width 0.2) (layer "F.Cu") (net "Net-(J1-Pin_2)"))
 (segment (start 81.8275 60.035) (end 89.5 60.035) (width 0.3) (layer "F.Cu") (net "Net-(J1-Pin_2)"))
 (segment (start 140.5 93.5) (end 140.5 81) (width 0.3) (layer "F.Cu") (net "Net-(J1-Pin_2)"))
 (segment (start 75.5 65.5) (end 75.5 93.5) (width 0.3) (layer "F.Cu") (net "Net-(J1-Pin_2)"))
 (segment (start 89.5 60.035) (end 89.5 63.5) (width 0.3) (layer "F.Cu") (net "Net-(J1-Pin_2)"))
 (segment (start 157.955 86.045) (end 148.6725 86.045) (width 0.3) (layer "F.Cu") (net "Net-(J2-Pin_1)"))
 (segment (start 158 62.5) (end 158 86) (width 0.3) (layer "F.Cu") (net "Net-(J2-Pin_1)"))
 (segment (start 158 86) (end 157.955 86.045) (width 0.2) (layer "F.Cu") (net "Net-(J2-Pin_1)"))
 (segment (start 155.5 60) (end 158 62.5) (width 0.3) (layer "F.Cu") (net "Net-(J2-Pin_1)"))
 (segment (start 150.1 60) (end 155.5 60) (width 0.3) (layer "F.Cu") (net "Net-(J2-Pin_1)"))
 (segment (start 130.59 73.5) (end 132.5 75.41) (width 0.2) (layer "F.Cu") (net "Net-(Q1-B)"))
 (segment (start 114.69 76) (end 114.69 73.81) (width 0.2) (layer "F.Cu") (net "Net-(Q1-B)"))
 (segment (start 114.69 73.81) (end 115 73.5) (width 0.2) (layer "F.Cu") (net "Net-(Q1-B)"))
 (segment (start 115 73.5) (end 130.59 73.5) (width 0.2) (layer "F.Cu") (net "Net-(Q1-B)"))
 (segment (start 132.5 75.41) (end 132.5 76.36) (width 0.2) (layer "F.Cu") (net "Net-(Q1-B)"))
 (segment (start 103.6 77.1) (end 101.38 74.88) (width 0.2) (layer "F.Cu") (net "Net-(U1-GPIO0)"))
 (segment (start 124.85 76) (end 123.75 77.1) (width 0.2) (layer "F.Cu") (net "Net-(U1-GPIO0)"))
 (segment (start 123.75 77.1) (end 103.6 77.1) (width 0.2) (layer "F.Cu") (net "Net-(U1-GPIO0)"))
 (segment (start 111.42 90) (end 116.27 90) (width 0.2) (layer "F.Cu") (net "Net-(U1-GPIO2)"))
 (segment (start 116.27 90) (end 122.77 90) (width 0.2) (layer "F.Cu") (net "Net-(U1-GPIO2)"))
 (segment (start 96.3 74.88) (end 111.42 90) (width 0.2) (layer "F.Cu") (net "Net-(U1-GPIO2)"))
 (segment (start 86.14 74.88) (end 95.02 66) (width 0.2) (layer "F.Cu") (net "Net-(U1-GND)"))
 (segment (start 111.0925 64.4) (end 124.2925 51.2) (width 0.2) (layer "F.Cu") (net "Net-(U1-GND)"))
 (segment (start 124.2925 51.2) (end 124.2925 50) (width 0.2) (layer "F.Cu") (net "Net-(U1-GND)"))
 (segment (start 107.5 64.4) (end 111.0925 64.4) (width 0.2) (layer "F.Cu") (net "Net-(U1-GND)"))
 (segment (start 95.02 66) (end 106 66) (width 0.2) (layer "F.Cu") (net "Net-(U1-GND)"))
 (via (at 107.5 64.4) (size 0.6) (drill 0.3) (layers "F.Cu" "B.Cu") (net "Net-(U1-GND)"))
 (via (at 106 66) (size 0.6) (drill 0.3) (layers "F.Cu" "B.Cu") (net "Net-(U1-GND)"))
 (segment (start 107.5 64.5) (end 107.5 64.4) (width 0.2) (layer "B.Cu") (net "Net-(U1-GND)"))
 (segment (start 106 66) (end 107.5 64.5) (width 0.2) (layer "B.Cu") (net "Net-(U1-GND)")))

